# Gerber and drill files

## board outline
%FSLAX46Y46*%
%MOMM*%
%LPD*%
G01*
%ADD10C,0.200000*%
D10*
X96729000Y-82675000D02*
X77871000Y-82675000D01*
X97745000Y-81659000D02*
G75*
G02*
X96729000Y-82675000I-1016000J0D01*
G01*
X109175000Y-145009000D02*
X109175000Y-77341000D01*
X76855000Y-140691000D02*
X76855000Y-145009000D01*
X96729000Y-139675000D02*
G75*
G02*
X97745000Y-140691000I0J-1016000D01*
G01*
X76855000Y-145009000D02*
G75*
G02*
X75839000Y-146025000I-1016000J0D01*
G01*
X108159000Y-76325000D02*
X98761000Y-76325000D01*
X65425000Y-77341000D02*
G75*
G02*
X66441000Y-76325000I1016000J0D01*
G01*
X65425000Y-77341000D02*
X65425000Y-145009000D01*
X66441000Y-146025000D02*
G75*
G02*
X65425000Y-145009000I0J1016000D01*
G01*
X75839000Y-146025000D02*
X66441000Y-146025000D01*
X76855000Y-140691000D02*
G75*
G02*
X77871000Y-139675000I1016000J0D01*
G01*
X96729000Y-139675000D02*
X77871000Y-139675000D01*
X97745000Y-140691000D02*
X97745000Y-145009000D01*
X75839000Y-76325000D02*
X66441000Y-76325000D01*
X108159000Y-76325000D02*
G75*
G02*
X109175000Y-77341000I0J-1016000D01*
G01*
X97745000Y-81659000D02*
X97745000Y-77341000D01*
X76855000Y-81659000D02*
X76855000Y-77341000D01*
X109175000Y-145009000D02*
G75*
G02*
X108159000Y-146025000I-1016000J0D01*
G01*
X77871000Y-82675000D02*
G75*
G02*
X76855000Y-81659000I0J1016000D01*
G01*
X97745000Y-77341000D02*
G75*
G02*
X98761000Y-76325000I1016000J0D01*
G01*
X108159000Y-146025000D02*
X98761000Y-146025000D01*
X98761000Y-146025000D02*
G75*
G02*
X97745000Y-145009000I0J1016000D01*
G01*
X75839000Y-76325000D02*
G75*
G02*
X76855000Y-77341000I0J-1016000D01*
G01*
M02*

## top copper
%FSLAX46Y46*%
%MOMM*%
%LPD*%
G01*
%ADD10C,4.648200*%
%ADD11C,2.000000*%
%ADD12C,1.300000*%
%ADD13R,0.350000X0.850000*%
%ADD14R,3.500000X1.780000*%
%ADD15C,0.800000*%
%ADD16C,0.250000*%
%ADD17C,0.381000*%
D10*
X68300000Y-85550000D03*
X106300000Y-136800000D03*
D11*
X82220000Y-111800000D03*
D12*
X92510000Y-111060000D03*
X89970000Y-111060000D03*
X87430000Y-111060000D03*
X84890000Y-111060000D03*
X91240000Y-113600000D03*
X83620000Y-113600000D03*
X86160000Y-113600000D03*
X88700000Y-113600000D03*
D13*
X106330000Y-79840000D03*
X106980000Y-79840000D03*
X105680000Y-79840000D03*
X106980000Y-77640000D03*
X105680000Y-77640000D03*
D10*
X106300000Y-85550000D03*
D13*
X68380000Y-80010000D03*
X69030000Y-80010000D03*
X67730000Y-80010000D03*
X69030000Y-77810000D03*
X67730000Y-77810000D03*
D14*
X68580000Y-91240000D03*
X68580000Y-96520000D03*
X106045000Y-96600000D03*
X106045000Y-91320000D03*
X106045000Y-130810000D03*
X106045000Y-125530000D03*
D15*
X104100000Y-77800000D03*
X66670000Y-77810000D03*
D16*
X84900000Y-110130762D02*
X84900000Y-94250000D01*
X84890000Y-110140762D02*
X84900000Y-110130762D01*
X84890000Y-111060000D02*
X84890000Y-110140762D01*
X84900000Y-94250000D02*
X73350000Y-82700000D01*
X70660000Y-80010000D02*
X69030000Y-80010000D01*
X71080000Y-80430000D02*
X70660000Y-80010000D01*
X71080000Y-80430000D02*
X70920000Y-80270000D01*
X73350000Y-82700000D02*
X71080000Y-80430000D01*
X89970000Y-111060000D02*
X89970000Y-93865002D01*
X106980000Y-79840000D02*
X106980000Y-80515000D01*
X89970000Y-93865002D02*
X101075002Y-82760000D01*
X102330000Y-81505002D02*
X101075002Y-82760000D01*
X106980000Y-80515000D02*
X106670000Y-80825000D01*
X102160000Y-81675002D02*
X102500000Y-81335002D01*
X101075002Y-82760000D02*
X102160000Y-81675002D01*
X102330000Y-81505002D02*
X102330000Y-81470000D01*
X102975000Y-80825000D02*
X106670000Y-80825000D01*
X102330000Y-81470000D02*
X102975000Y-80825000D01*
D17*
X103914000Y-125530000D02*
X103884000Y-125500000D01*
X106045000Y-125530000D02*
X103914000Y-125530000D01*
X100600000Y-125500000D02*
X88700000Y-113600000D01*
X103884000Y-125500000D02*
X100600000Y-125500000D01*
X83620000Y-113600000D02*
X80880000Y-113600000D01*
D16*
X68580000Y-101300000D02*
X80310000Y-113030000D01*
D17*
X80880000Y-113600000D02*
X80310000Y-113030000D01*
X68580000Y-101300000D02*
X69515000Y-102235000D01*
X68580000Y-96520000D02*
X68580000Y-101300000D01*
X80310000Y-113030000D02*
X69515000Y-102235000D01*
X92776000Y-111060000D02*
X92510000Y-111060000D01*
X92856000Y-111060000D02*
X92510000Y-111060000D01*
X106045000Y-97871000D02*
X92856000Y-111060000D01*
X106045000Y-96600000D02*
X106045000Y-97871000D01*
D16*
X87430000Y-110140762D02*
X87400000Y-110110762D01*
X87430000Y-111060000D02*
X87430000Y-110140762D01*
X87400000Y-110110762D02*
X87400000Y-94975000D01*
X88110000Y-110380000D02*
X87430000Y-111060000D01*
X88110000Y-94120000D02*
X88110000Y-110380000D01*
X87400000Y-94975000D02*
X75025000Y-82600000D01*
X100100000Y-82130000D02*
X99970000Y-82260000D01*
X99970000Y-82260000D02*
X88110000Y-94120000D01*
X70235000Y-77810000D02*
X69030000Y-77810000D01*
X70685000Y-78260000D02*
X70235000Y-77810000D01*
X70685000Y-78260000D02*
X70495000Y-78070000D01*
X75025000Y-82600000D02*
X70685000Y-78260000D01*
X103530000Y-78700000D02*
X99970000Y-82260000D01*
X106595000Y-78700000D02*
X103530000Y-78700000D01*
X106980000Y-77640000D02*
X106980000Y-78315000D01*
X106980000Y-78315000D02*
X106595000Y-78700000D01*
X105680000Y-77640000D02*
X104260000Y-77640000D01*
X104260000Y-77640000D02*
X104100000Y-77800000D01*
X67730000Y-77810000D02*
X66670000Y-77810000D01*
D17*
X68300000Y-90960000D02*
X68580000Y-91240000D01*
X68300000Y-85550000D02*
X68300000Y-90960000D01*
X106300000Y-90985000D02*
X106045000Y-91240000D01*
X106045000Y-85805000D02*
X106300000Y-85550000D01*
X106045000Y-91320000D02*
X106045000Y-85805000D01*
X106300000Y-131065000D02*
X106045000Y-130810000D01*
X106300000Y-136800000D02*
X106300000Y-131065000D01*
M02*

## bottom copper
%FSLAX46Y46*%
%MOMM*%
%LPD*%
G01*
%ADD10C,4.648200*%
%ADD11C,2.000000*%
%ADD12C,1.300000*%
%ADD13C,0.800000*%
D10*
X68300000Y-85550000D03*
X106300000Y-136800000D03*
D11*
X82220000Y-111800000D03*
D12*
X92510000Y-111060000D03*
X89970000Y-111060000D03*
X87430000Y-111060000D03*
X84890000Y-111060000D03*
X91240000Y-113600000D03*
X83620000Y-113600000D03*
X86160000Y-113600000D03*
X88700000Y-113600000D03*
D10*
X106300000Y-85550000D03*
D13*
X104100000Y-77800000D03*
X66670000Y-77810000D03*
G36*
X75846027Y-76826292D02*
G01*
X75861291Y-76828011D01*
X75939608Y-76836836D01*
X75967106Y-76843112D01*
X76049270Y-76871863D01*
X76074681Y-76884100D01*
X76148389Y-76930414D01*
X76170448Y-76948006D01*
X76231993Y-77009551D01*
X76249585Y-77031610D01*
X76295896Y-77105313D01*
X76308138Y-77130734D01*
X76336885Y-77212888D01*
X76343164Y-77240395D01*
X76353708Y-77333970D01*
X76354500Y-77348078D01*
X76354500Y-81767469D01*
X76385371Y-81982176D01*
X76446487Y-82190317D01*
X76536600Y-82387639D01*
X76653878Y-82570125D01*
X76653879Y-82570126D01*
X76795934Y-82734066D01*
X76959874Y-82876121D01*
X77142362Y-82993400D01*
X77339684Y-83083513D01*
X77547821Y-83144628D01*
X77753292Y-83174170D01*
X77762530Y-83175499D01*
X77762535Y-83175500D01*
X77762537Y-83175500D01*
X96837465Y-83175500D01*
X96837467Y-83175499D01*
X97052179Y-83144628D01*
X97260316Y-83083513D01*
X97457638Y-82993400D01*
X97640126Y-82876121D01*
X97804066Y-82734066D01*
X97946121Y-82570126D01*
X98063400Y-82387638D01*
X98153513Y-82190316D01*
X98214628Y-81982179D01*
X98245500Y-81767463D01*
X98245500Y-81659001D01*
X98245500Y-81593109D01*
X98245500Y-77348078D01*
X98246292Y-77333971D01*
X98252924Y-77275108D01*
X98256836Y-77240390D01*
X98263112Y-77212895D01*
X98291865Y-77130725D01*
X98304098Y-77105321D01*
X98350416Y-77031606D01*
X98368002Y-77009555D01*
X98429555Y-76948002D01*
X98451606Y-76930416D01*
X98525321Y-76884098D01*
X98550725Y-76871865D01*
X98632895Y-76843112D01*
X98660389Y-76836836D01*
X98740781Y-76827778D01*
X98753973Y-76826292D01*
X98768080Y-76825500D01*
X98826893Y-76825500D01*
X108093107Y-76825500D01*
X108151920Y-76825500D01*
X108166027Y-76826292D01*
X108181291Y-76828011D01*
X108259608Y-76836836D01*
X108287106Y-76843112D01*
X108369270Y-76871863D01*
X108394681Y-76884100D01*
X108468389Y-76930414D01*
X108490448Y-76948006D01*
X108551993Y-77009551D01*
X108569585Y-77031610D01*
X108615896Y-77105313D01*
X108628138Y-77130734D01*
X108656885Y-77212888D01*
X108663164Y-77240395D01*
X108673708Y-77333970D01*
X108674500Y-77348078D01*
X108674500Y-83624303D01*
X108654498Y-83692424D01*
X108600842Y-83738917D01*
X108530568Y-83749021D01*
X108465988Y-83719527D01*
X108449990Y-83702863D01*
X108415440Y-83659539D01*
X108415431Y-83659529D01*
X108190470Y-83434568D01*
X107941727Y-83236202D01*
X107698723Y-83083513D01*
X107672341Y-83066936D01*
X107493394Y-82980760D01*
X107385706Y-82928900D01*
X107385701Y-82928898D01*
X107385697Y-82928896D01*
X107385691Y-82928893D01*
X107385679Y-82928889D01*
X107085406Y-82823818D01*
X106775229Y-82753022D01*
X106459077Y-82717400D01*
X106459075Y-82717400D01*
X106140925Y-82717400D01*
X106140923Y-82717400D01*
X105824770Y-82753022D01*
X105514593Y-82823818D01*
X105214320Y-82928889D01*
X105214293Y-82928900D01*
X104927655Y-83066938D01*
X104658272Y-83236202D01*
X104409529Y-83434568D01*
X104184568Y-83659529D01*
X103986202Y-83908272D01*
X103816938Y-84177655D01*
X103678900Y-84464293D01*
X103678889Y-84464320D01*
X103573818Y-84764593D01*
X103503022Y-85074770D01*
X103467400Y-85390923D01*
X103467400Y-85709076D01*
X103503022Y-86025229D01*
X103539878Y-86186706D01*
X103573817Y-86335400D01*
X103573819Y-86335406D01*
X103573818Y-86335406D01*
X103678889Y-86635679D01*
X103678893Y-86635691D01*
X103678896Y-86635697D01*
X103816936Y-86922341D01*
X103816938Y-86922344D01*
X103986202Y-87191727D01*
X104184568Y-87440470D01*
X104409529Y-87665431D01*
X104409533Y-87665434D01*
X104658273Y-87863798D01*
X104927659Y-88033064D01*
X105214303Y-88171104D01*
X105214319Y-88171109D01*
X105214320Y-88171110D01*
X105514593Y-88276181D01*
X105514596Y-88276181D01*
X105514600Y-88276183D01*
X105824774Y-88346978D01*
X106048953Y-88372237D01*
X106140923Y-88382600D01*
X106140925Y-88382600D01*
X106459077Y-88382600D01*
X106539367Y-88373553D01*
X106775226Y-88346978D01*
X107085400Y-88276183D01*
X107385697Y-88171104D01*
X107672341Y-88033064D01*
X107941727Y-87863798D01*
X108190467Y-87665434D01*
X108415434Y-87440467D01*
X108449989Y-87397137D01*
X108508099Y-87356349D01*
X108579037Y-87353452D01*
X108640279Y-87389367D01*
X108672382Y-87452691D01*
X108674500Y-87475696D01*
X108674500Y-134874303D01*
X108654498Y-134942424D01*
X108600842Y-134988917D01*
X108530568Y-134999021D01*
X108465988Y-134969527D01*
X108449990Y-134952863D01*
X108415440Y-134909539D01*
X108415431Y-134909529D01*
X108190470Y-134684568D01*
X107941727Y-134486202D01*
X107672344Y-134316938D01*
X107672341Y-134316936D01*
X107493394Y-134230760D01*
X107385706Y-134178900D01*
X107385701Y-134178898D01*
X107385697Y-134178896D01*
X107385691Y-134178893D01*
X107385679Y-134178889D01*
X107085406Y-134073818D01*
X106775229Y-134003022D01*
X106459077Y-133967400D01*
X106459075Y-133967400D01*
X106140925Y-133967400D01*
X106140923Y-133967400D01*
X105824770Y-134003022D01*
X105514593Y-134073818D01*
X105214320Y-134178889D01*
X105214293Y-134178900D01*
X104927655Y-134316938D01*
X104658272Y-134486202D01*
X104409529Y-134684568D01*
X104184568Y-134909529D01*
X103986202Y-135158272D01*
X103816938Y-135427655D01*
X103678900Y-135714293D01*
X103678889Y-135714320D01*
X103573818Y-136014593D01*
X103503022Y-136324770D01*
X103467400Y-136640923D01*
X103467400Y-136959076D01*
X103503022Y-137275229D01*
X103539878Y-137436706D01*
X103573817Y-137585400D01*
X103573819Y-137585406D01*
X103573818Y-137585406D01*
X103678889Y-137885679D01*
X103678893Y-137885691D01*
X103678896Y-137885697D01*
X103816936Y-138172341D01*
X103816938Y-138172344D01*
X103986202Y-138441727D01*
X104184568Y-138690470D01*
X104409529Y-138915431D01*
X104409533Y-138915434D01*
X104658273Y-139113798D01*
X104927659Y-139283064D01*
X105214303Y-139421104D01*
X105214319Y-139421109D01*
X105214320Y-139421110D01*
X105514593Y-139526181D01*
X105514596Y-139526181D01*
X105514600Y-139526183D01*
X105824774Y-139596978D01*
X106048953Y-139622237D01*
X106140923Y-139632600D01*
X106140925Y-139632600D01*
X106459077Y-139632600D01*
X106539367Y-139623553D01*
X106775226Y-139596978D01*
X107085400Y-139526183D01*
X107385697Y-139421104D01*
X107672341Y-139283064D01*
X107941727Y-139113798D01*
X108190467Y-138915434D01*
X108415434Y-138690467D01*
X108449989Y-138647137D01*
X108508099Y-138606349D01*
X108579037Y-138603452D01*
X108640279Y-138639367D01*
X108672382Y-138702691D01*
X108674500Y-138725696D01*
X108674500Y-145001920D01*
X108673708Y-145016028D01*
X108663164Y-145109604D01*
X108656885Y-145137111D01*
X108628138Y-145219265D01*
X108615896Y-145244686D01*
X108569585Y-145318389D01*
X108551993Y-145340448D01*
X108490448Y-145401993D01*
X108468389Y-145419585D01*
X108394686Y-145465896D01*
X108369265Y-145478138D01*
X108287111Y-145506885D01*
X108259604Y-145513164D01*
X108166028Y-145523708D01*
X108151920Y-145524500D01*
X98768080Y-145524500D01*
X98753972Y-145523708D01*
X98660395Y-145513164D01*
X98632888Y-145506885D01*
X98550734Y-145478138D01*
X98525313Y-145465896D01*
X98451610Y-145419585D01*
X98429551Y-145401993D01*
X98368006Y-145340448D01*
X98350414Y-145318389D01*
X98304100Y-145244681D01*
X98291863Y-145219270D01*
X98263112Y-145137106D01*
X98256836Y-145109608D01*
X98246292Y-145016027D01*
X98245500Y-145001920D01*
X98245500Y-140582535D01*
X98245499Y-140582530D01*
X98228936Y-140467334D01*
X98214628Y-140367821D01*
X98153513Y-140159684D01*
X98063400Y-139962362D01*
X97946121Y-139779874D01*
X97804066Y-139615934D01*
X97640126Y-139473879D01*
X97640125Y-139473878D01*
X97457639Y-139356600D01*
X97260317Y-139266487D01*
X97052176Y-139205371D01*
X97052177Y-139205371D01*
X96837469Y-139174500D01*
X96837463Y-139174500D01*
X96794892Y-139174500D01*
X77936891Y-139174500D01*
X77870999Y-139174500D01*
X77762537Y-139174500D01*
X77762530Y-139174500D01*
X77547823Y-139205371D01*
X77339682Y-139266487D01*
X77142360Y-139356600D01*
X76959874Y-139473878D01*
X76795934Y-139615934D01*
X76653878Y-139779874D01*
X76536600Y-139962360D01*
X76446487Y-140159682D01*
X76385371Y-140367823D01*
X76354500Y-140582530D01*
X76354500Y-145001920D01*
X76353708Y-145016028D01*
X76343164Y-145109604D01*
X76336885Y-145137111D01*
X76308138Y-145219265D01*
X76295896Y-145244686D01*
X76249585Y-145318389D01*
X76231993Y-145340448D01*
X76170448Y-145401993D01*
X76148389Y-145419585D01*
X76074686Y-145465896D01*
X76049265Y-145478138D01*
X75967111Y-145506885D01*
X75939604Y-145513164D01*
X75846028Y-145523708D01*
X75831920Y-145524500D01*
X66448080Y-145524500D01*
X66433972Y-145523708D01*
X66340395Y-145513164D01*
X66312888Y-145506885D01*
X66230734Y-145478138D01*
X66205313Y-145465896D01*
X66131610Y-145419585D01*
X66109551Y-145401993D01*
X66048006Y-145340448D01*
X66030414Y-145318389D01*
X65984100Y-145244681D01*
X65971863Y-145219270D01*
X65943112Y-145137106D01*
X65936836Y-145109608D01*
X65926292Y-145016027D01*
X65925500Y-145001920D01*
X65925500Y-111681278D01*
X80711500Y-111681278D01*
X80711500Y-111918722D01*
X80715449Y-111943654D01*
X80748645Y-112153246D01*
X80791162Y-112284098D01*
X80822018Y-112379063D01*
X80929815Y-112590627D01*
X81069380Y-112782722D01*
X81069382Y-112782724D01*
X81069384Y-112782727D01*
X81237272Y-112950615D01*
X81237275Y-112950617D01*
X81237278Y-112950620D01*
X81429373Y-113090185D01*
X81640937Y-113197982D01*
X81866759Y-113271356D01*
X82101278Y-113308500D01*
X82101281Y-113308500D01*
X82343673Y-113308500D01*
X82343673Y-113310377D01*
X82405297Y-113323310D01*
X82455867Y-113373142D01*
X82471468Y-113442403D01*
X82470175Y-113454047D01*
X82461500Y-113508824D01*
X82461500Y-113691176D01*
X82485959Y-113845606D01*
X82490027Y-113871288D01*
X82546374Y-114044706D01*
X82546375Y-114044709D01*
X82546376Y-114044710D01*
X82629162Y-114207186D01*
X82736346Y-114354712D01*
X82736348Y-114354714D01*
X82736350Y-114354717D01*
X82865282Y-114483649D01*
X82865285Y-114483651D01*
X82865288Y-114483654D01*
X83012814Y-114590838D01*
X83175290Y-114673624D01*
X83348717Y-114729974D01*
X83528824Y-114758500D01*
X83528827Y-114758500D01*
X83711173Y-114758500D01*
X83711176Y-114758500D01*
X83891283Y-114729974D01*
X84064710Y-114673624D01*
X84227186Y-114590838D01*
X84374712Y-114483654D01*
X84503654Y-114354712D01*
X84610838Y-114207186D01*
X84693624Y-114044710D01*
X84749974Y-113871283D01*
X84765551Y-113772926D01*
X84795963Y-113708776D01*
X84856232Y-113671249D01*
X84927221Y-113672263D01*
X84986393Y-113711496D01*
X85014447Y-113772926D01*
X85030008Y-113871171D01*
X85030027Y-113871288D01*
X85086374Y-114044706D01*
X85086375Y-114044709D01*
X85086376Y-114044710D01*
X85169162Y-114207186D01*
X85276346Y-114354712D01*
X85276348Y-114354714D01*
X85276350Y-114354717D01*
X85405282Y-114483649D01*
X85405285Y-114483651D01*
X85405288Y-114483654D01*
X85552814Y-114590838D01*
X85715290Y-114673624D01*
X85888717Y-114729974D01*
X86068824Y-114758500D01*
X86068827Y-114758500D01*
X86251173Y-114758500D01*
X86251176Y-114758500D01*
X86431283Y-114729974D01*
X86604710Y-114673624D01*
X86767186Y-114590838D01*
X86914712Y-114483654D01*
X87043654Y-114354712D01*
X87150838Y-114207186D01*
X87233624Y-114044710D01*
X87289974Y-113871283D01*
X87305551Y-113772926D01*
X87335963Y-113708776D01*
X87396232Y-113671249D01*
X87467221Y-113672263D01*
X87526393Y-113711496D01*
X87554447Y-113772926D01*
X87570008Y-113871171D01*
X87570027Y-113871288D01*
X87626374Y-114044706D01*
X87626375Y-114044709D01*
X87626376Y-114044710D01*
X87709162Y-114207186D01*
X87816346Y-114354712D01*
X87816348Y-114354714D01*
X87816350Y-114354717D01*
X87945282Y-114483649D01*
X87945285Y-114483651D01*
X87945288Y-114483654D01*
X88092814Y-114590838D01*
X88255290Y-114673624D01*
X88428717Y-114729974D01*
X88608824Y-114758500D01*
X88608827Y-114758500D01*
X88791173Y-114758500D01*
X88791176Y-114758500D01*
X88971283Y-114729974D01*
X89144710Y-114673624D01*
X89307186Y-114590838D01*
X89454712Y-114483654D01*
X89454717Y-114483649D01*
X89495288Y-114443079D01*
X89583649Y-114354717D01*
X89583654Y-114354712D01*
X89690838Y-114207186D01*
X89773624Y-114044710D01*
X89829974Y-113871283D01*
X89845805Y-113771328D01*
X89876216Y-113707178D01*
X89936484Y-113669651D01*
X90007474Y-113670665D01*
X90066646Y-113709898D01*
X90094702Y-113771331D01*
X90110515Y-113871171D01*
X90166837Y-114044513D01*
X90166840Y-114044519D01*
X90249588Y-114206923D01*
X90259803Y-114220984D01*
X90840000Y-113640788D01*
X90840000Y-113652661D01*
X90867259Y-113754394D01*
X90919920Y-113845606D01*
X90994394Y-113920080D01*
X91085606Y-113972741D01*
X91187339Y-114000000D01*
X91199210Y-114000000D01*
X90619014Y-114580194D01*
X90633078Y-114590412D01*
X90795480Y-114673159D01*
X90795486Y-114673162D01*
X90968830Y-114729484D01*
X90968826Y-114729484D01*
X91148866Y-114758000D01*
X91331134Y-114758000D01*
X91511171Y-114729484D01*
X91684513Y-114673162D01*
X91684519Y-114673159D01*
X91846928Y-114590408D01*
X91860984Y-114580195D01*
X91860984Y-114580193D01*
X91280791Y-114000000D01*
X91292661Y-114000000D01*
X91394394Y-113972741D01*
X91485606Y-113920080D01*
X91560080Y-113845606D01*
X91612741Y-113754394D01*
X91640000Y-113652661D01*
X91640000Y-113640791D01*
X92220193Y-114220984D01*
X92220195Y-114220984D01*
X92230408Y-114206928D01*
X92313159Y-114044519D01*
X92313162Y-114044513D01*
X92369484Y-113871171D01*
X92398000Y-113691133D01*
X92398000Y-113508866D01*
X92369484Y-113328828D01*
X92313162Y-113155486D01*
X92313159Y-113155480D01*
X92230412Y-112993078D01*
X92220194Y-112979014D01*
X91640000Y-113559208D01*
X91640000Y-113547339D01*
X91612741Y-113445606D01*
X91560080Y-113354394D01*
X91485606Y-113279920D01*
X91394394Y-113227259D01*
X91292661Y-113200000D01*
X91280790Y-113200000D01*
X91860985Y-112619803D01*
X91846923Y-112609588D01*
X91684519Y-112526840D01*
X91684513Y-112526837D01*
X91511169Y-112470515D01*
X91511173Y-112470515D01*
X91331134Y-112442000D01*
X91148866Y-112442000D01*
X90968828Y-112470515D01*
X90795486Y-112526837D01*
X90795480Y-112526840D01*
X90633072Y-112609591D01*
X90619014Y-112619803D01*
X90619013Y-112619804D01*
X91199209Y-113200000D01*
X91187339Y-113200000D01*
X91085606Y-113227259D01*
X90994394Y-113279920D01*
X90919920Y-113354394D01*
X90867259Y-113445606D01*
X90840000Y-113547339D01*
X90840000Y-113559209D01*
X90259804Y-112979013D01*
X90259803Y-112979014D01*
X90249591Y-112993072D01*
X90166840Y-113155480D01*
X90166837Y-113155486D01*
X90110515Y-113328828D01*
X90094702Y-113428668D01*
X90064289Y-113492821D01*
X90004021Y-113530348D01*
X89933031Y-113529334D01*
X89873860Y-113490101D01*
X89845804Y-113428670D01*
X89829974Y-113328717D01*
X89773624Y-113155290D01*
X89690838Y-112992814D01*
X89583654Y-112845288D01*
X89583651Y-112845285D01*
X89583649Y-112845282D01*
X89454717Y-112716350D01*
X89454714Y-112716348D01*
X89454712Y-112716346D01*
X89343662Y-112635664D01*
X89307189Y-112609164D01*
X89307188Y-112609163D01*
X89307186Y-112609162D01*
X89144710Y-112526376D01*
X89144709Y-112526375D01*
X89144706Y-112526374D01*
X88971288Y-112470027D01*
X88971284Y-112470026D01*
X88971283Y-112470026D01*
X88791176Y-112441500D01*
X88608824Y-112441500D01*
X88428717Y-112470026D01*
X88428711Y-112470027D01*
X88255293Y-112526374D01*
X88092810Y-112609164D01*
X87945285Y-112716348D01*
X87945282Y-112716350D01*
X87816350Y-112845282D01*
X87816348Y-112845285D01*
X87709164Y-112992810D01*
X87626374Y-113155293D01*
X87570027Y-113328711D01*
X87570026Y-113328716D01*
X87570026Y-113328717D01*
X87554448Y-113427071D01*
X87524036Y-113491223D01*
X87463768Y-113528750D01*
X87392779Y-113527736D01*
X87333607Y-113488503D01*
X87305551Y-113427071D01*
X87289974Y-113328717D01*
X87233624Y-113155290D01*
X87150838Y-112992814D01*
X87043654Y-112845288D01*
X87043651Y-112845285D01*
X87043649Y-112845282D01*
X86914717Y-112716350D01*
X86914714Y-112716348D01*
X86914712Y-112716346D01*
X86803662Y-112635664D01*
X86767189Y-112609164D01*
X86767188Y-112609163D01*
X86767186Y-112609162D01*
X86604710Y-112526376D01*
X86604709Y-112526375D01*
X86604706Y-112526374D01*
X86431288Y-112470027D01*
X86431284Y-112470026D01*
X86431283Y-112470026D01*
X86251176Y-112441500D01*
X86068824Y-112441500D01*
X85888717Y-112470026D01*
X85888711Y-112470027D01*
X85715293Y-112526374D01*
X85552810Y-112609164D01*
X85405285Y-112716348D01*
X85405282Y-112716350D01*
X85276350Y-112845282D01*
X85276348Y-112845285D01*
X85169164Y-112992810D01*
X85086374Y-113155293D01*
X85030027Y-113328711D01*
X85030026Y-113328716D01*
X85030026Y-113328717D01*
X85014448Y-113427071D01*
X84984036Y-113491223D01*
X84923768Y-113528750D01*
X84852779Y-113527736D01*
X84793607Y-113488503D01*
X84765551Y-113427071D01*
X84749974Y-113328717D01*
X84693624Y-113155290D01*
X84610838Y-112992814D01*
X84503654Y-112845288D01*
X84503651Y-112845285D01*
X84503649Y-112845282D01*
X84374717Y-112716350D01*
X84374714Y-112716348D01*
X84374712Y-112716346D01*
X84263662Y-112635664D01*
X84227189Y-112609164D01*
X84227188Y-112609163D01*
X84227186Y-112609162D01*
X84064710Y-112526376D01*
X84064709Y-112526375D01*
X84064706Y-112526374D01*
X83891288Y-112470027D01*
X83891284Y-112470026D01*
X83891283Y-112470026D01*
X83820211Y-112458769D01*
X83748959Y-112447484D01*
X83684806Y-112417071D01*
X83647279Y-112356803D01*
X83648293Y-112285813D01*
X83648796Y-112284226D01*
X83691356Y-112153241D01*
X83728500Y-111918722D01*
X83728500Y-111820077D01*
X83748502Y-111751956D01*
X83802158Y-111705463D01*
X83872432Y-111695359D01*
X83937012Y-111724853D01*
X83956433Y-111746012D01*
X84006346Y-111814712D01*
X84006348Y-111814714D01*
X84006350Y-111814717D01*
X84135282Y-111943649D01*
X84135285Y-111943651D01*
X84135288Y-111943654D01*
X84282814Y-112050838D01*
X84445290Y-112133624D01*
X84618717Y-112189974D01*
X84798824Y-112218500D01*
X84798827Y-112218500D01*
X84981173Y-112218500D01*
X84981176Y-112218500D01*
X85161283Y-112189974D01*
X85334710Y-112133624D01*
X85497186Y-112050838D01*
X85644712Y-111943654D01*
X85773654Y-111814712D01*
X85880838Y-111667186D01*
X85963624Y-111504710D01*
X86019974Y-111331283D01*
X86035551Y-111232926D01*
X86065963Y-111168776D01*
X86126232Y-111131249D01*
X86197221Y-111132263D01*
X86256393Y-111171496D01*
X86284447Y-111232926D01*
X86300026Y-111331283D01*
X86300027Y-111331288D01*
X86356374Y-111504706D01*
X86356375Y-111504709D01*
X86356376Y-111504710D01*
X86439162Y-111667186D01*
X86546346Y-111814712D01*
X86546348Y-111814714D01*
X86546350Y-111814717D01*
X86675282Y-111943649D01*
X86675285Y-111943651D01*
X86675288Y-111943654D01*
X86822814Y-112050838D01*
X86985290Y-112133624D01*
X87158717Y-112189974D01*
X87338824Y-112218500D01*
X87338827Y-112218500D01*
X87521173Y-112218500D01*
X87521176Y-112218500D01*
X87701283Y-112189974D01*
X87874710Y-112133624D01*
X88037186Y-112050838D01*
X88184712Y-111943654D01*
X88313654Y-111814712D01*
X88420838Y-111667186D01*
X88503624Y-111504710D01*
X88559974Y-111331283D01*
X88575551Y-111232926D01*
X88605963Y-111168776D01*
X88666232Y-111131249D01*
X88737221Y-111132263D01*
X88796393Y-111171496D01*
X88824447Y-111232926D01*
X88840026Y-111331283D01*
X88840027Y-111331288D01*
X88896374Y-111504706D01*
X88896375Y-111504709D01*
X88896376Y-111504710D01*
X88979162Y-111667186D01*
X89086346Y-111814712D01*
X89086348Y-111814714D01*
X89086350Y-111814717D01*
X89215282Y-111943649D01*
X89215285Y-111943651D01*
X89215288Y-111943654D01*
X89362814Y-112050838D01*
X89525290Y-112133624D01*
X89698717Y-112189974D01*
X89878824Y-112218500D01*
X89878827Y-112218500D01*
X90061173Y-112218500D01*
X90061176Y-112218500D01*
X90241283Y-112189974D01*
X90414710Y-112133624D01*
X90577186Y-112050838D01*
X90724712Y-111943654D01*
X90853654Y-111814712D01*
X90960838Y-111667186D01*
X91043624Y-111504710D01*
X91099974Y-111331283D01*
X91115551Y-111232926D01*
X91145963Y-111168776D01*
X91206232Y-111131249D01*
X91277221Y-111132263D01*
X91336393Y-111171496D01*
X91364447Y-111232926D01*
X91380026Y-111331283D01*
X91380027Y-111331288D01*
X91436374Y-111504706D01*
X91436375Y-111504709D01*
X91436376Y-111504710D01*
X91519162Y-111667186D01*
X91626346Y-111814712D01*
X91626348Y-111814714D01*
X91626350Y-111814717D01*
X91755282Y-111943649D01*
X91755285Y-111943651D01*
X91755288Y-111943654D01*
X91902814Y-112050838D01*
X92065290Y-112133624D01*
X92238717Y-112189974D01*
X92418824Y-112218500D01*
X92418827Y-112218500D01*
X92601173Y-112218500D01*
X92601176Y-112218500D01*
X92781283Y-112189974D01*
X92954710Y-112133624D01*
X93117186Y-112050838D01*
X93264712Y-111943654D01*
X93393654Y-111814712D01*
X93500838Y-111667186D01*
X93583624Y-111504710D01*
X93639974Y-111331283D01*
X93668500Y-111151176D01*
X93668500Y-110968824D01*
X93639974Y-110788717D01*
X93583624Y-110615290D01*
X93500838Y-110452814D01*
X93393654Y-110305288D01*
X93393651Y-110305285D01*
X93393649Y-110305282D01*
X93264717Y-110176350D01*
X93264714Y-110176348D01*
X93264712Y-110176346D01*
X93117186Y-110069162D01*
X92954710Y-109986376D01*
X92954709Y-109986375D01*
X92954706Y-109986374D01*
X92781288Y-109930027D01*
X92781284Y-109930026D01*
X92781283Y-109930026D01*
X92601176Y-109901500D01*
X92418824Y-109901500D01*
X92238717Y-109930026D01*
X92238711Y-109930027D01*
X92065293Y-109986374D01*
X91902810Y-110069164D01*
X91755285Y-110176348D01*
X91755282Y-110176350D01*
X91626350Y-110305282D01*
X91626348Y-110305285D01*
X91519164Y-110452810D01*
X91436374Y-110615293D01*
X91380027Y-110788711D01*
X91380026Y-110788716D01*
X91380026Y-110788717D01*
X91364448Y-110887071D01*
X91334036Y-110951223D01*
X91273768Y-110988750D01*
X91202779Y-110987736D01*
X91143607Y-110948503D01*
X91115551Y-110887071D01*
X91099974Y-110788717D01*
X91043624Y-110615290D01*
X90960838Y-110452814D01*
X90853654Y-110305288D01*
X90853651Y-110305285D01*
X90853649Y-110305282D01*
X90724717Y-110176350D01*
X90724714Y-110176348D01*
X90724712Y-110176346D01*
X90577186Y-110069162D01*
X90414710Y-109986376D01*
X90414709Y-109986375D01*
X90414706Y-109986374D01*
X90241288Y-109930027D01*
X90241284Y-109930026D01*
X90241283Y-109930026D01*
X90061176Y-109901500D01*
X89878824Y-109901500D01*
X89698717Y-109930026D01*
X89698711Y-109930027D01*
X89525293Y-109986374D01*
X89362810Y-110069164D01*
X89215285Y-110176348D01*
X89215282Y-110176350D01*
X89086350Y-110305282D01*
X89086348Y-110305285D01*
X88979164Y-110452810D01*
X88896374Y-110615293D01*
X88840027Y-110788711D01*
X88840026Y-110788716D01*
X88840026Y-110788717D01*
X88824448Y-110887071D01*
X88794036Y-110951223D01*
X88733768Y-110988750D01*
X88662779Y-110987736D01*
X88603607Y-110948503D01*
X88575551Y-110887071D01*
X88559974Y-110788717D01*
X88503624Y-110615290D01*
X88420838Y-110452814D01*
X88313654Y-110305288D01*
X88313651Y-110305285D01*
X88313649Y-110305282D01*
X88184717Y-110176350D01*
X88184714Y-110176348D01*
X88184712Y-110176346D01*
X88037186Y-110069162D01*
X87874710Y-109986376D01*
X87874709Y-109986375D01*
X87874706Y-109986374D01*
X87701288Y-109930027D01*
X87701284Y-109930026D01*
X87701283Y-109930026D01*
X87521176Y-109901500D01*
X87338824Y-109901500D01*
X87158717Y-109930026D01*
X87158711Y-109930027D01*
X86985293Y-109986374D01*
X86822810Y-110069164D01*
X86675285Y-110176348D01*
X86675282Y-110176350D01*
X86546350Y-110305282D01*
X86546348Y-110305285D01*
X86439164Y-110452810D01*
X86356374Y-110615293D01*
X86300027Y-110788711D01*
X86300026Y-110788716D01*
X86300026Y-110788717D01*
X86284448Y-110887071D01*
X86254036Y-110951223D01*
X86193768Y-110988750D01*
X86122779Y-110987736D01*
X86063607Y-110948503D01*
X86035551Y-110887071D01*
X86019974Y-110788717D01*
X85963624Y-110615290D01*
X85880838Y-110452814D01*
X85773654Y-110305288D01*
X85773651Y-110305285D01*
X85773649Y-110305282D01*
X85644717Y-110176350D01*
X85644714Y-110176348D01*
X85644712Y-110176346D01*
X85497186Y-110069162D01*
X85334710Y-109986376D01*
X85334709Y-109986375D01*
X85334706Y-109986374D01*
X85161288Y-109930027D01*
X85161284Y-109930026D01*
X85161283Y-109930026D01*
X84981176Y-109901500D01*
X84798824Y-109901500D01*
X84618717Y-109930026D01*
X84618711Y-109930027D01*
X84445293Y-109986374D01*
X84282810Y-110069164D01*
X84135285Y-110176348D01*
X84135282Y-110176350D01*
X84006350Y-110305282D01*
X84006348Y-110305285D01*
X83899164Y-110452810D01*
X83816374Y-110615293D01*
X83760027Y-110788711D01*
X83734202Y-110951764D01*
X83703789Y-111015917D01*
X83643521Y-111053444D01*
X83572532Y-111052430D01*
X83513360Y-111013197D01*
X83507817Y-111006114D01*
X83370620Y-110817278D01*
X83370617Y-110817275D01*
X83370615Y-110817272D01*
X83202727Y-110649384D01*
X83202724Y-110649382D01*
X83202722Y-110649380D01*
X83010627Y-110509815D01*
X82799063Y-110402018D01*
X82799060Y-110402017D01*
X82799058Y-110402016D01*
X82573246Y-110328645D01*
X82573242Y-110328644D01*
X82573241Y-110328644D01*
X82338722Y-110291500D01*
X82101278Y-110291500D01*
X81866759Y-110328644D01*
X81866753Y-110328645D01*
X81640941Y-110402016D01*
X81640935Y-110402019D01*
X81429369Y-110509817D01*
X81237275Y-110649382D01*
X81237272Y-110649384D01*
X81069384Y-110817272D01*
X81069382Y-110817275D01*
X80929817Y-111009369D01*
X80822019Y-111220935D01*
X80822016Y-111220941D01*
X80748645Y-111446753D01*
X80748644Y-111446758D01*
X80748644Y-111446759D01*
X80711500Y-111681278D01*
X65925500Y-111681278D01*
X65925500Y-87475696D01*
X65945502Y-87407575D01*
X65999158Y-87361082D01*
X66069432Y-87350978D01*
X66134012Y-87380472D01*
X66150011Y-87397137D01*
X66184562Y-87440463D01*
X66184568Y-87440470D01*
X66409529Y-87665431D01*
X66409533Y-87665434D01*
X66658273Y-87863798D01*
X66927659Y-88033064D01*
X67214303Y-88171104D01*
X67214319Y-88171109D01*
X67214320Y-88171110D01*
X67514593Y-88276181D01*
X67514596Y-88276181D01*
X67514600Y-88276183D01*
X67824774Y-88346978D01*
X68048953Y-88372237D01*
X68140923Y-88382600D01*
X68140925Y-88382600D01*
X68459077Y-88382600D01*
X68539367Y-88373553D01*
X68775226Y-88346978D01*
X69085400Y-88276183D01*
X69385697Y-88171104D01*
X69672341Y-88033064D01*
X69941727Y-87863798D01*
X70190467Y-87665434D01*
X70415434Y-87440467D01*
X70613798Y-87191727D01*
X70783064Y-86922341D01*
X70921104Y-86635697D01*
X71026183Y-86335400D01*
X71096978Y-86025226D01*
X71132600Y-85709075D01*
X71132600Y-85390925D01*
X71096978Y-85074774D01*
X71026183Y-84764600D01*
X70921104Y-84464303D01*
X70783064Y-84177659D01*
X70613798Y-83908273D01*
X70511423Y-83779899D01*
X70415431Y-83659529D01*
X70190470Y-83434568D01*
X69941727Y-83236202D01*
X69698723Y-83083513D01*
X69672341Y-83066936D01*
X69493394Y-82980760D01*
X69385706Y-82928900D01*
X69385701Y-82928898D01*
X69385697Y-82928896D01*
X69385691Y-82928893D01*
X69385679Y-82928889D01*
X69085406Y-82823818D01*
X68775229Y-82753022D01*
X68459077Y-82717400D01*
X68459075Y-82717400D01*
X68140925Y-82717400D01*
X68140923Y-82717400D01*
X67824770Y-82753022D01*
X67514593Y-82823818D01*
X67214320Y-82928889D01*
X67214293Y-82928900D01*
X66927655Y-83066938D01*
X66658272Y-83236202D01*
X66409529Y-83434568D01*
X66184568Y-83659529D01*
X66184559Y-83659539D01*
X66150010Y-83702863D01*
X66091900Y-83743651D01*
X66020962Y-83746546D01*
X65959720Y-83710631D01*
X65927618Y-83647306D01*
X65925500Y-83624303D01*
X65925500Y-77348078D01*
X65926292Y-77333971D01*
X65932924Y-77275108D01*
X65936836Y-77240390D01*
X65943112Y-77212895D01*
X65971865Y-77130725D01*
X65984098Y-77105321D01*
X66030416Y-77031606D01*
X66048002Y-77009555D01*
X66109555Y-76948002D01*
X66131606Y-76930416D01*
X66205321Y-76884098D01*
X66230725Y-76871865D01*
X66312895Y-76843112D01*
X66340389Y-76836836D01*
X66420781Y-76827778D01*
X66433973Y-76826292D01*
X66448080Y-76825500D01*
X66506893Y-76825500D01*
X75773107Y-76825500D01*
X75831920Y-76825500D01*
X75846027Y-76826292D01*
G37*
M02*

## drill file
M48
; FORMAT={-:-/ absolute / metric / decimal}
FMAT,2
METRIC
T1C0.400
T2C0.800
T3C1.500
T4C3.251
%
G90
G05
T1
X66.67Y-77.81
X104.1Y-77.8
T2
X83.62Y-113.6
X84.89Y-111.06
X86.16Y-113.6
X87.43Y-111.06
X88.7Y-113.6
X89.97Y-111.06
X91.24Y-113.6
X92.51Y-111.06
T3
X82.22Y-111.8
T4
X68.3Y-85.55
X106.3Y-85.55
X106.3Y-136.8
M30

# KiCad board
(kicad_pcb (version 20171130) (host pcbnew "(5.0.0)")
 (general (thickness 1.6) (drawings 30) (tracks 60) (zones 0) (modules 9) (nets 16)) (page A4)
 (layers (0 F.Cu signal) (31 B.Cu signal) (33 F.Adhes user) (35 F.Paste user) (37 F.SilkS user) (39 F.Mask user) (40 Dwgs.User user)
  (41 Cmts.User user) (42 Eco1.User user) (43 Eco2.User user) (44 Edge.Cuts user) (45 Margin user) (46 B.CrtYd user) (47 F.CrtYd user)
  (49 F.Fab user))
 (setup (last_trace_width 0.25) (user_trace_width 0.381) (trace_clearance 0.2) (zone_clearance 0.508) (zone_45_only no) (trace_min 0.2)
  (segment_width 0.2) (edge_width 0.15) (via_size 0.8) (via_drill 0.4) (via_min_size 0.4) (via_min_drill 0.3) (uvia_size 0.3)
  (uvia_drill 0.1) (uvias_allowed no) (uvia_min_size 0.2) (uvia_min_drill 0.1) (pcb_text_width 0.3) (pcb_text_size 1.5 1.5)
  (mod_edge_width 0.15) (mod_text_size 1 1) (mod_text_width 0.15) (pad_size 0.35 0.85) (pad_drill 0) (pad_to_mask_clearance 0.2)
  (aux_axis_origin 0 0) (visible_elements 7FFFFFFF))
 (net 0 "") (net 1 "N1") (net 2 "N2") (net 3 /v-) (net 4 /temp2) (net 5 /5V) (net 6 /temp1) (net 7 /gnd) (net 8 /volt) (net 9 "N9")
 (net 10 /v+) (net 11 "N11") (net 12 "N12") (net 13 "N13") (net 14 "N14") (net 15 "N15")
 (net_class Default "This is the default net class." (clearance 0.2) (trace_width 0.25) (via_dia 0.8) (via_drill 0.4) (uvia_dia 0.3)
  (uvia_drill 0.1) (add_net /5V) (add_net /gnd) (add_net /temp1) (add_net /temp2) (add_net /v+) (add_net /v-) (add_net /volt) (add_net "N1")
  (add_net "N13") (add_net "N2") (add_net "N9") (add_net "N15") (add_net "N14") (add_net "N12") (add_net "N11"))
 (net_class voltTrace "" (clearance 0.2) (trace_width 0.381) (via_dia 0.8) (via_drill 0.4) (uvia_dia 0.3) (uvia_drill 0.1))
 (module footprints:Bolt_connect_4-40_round (layer F.Cu) (at 68.3 85.55)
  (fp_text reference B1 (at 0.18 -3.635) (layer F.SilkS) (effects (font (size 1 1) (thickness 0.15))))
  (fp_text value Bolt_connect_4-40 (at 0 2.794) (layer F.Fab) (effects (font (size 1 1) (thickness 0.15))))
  (pad 1 thru_hole circle (at 0 0) (size 4.6482 4.6482) (drill 3.2512) (layers *.Cu *.Mask) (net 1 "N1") (clearance 0.508)))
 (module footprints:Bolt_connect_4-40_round (layer F.Cu) (at 106.3 136.8)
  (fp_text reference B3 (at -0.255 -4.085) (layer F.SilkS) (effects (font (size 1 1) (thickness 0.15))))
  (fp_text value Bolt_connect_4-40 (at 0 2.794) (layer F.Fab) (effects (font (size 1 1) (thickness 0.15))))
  (pad 1 thru_hole circle (at 0 0) (size 4.6482 4.6482) (drill 3.2512) (layers *.Cu *.Mask) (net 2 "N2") (clearance 0.508)))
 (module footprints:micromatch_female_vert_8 (layer F.Cu) (at 88.7 113.6 90)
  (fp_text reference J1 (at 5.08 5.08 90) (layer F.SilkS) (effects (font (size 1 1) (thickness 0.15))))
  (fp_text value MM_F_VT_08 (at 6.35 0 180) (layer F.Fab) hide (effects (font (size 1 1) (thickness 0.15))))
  (pad 9 thru_hole circle (at 1.8 -6.48 90) (size 2 2) (drill 1.5) (layers *.Cu *.Mask))
  (pad 8 thru_hole circle (at 2.54 3.81 90) (size 1.3 1.3) (drill 0.8) (layers *.Cu *.Mask) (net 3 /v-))
  (pad 6 thru_hole circle (at 2.54 1.27 90) (size 1.3 1.3) (drill 0.8) (layers *.Cu *.Mask) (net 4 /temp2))
  (pad 4 thru_hole circle (at 2.54 -1.27 90) (size 1.3 1.3) (drill 0.8) (layers *.Cu *.Mask) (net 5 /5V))
  (pad 2 thru_hole circle (at 2.54 -3.81 90) (size 1.3 1.3) (drill 0.8) (layers *.Cu *.Mask) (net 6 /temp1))
  (pad 7 thru_hole circle (at 0 2.54 90) (size 1.3 1.3) (drill 0.8) (layers *.Cu *.Mask) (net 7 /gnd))
  (pad 1 thru_hole circle (at 0 -5.08 90) (size 1.3 1.3) (drill 0.8) (layers *.Cu *.Mask) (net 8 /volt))
  (pad 3 thru_hole circle (at 0 -2.54 90) (size 1.3 1.3) (drill 0.8) (layers *.Cu *.Mask) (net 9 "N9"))
  (pad 5 thru_hole circle (at 0 0 90) (size 1.3 1.3) (drill 0.8) (layers *.Cu *.Mask) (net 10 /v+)))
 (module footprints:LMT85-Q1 (layer F.Cu) (at 105.68 79.84)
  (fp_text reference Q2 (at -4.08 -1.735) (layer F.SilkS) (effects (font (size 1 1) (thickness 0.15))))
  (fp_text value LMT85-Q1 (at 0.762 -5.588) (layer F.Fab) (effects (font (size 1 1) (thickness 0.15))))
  (pad 3 smd rect (at 0.65 0) (size 0.35 0.85) (layers F.Cu F.Paste F.Mask) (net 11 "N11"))
  (pad 4 smd rect (at 1.3 0) (size 0.35 0.85) (layers F.Cu F.Paste F.Mask) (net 4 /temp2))
  (pad 2 smd rect (at 0 0) (size 0.35 0.85) (layers F.Cu F.Paste F.Mask) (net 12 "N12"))
  (pad 5 smd rect (at 1.3 -2.2) (size 0.35 0.85) (layers F.Cu F.Paste F.Mask) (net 5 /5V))
  (pad 1 smd rect (at 0 -2.2) (size 0.35 0.85) (layers F.Cu F.Paste F.Mask) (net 7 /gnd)))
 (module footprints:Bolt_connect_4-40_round (layer F.Cu) (at 106.3 85.55)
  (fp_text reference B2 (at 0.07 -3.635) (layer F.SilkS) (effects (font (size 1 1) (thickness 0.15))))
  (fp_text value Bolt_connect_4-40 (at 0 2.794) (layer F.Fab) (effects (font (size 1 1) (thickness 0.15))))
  (pad 1 thru_hole circle (at 0 0) (size 4.6482 4.6482) (drill 3.2512) (layers *.Cu *.Mask) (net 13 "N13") (clearance 0.508)))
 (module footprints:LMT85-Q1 (layer F.Cu) (at 67.73 80.01)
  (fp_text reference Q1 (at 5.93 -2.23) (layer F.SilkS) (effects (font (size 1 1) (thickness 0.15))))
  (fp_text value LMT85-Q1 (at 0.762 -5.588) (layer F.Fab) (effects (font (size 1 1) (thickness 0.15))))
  (pad 3 smd rect (at 0.65 0) (size 0.35 0.85) (layers F.Cu F.Paste F.Mask) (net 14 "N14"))
  (pad 4 smd rect (at 1.3 0) (size 0.35 0.85) (layers F.Cu F.Paste F.Mask) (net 6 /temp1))
  (pad 2 smd rect (at 0 0) (size 0.35 0.85) (layers F.Cu F.Paste F.Mask) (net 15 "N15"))
  (pad 5 smd rect (at 1.3 -2.2) (size 0.35 0.85) (layers F.Cu F.Paste F.Mask) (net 5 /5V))
  (pad 1 smd rect (at 0 -2.2) (size 0.35 0.85) (layers F.Cu F.Paste F.Mask) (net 7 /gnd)))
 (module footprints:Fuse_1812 (layer F.Cu) (at 68.58 96.52 90)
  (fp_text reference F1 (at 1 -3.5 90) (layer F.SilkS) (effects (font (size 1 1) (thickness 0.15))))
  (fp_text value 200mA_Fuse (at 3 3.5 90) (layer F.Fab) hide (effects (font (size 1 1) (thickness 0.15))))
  (pad 2 smd rect (at 5.28 0 90) (size 1.78 3.5) (layers F.Cu F.Paste F.Mask) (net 1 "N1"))
  (pad 1 smd rect (at 0 0 90) (size 1.78 3.5) (layers F.Cu F.Paste F.Mask) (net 8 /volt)))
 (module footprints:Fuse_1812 (layer F.Cu) (at 106.045 96.6 90)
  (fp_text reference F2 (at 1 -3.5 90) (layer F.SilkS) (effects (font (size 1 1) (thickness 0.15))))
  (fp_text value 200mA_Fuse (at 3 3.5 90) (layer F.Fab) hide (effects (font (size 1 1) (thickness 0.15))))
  (pad 1 smd rect (at 0 0 90) (size 1.78 3.5) (layers F.Cu F.Paste F.Mask) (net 3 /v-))
  (pad 2 smd rect (at 5.28 0 90) (size 1.78 3.5) (layers F.Cu F.Paste F.Mask) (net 13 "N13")))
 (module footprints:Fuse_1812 (layer F.Cu) (at 106.045 125.53 270)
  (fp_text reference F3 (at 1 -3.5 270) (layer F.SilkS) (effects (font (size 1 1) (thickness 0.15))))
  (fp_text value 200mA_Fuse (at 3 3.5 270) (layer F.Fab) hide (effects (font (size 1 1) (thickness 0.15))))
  (pad 2 smd rect (at 5.28 0 270) (size 1.78 3.5) (layers F.Cu F.Paste F.Mask) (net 2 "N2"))
  (pad 1 smd rect (at 0 0 270) (size 1.78 3.5) (layers F.Cu F.Paste F.Mask) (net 10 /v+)))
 (gr_line (start 96.729 82.675) (end 77.871 82.675) (layer Edge.Cuts) (width 0.2))
 (gr_arc (start 96.729 81.659) (end 96.729 82.675) (angle -90) (layer Edge.Cuts) (width 0.2))
 (gr_line (start 109.175 145.009) (end 109.175 77.341) (layer Edge.Cuts) (width 0.2))
 (gr_line (start 76.855 140.691) (end 76.855 145.009) (layer Edge.Cuts) (width 0.2))
 (gr_arc (start 96.729 140.691) (end 97.745 140.691) (angle -90) (layer Edge.Cuts) (width 0.2))
 (gr_arc (start 75.839 145.009) (end 75.839 146.025) (angle -90) (layer Edge.Cuts) (width 0.2))
 (gr_line (start 108.159 76.325) (end 98.761 76.325) (layer Edge.Cuts) (width 0.2))
 (gr_arc (start 66.441 77.341) (end 66.441 76.325) (angle -90) (layer Edge.Cuts) (width 0.2))
 (gr_line (start 65.425 77.341) (end 65.425 145.009) (layer Edge.Cuts) (width 0.2))
 (gr_arc (start 66.441 145.009) (end 65.425 145.009) (angle -90) (layer Edge.Cuts) (width 0.2))
 (gr_line (start 75.839 146.025) (end 66.441 146.025) (layer Edge.Cuts) (width 0.2))
 (gr_arc (start 77.871 140.691) (end 77.871 139.675) (angle -90) (layer Edge.Cuts) (width 0.2))
 (gr_line (start 96.729 139.675) (end 77.871 139.675) (layer Edge.Cuts) (width 0.2))
 (gr_line (start 97.745 140.691) (end 97.745 145.009) (layer Edge.Cuts) (width 0.2))
 (gr_line (start 75.839 76.325) (end 66.441 76.325) (layer Edge.Cuts) (width 0.2))
 (gr_arc (start 108.159 77.341) (end 109.175 77.341) (angle -90) (layer Edge.Cuts) (width 0.2))
 (gr_line (start 97.745 81.659) (end 97.745 77.341) (layer Edge.Cuts) (width 0.2))
 (gr_line (start 76.855 81.659) (end 76.855 77.341) (layer Edge.Cuts) (width 0.2))
 (gr_arc (start 108.159 145.009) (end 108.159 146.025) (angle -90) (layer Edge.Cuts) (width 0.2))
 (gr_arc (start 77.871 81.659) (end 76.855 81.659) (angle -90) (layer Edge.Cuts) (width 0.2))
 (gr_arc (start 98.761 77.341) (end 98.761 76.325) (angle -90) (layer Edge.Cuts) (width 0.2))
 (gr_line (start 108.159 146.025) (end 98.761 146.025) (layer Edge.Cuts) (width 0.2))
 (gr_arc (start 98.761 145.009) (end 97.745 145.009) (angle -90) (layer Edge.Cuts) (width 0.2))
 (gr_arc (start 75.839 77.341) (end 76.855 77.341) (angle -90) (layer Edge.Cuts) (width 0.2))
 (segment (start 84.9 110.130762) (end 84.9 94.25) (width 0.25) (layer F.Cu) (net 6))
 (segment (start 84.89 110.140762) (end 84.9 110.130762) (width 0.25) (layer F.Cu) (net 6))
 (segment (start 84.89 111.06) (end 84.89 110.140762) (width 0.25) (layer F.Cu) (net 6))
 (segment (start 84.9 94.25) (end 73.35 82.7) (width 0.25) (layer F.Cu) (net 6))
 (segment (start 70.66 80.01) (end 69.03 80.01) (width 0.25) (layer F.Cu) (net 6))
 (segment (start 71.08 80.43) (end 70.66 80.01) (width 0.25) (layer F.Cu) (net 6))
 (segment (start 71.08 80.43) (end 70.92 80.27) (width 0.25) (layer F.Cu) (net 6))
 (segment (start 73.35 82.7) (end 71.08 80.43) (width 0.25) (layer F.Cu) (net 6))
 (segment (start 89.97 111.06) (end 89.97 93.865002) (width 0.25) (layer F.Cu) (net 4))
 (segment (start 106.98 79.84) (end 106.98 80.515) (width 0.25) (layer F.Cu) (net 4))
 (segment (start 89.97 93.865002) (end 101.075002 82.76) (width 0.25) (layer F.Cu) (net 4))
 (segment (start 102.33 81.505002) (end 101.075002 82.76) (width 0.25) (layer F.Cu) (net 4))
 (segment (start 106.98 80.515) (end 106.67 80.825) (width 0.25) (layer F.Cu) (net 4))
 (segment (start 102.16 81.675002) (end 102.5 81.335002) (width 0.25) (layer F.Cu) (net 4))
 (segment (start 101.075002 82.76) (end 102.16 81.675002) (width 0.25) (layer F.Cu) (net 4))
 (segment (start 102.33 81.505002) (end 102.33 81.47) (width 0.25) (layer F.Cu) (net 4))
 (segment (start 102.975 80.825) (end 106.67 80.825) (width 0.25) (layer F.Cu) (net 4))
 (segment (start 102.33 81.47) (end 102.975 80.825) (width 0.25) (layer F.Cu) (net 4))
 (segment (start 103.914 125.53) (end 103.884 125.5) (width 0.381) (layer F.Cu) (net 10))
 (segment (start 106.045 125.53) (end 103.914 125.53) (width 0.381) (layer F.Cu) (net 10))
 (segment (start 100.6 125.5) (end 88.7 113.6) (width 0.381) (layer F.Cu) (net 10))
 (segment (start 103.884 125.5) (end 100.6 125.5) (width 0.381) (layer F.Cu) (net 10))
 (segment (start 83.62 113.6) (end 80.88 113.6) (width 0.381) (layer F.Cu) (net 8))
 (segment (start 68.58 101.3) (end 80.31 113.03) (width 0.25) (layer F.Cu) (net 8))
 (segment (start 80.88 113.6) (end 80.31 113.03) (width 0.381) (layer F.Cu) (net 8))
 (segment (start 68.58 101.3) (end 69.515 102.235) (width 0.381) (layer F.Cu) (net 8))
 (segment (start 68.58 96.52) (end 68.58 101.3) (width 0.381) (layer F.Cu) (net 8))
 (segment (start 80.31 113.03) (end 69.515 102.235) (width 0.381) (layer F.Cu) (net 8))
 (segment (start 92.776 111.06) (end 92.51 111.06) (width 0.381) (layer F.Cu) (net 3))
 (segment (start 92.856 111.06) (end 92.51 111.06) (width 0.381) (layer F.Cu) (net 3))
 (segment (start 106.045 97.871) (end 92.856 111.06) (width 0.381) (layer F.Cu) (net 3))
 (segment (start 106.045 96.6) (end 106.045 97.871) (width 0.381) (layer F.Cu) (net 3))
 (segment (start 87.43 110.140762) (end 87.4 110.110762) (width 0.25) (layer F.Cu) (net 5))
 (segment (start 87.43 111.06) (end 87.43 110.140762) (width 0.25) (layer F.Cu) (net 5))
 (segment (start 87.4 110.110762) (end 87.4 94.975) (width 0.25) (layer F.Cu) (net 5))
 (segment (start 88.11 110.38) (end 87.43 111.06) (width 0.25) (layer F.Cu) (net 5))
 (segment (start 88.11 94.12) (end 88.11 110.38) (width 0.25) (layer F.Cu) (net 5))
 (segment (start 87.4 94.975) (end 75.025 82.6) (width 0.25) (layer F.Cu) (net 5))
 (segment (start 100.1 82.13) (end 99.97 82.26) (width 0.25) (layer F.Cu) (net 5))
 (segment (start 99.97 82.26) (end 88.11 94.12) (width 0.25) (layer F.Cu) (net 5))
 (segment (start 70.235 77.81) (end 69.03 77.81) (width 0.25) (layer F.Cu) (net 5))
 (segment (start 70.685 78.26) (end 70.235 77.81) (width 0.25) (layer F.Cu) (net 5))
 (segment (start 70.685 78.26) (end 70.495 78.07) (width 0.25) (layer F.Cu) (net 5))
 (segment (start 75.025 82.6) (end 70.685 78.26) (width 0.25) (layer F.Cu) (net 5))
 (segment (start 103.53 78.7) (end 99.97 82.26) (width 0.25) (layer F.Cu) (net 5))
 (segment (start 106.595 78.7) (end 103.53 78.7) (width 0.25) (layer F.Cu) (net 5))
 (segment (start 106.98 77.64) (end 106.98 78.315) (width 0.25) (layer F.Cu) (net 5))
 (segment (start 106.98 78.315) (end 106.595 78.7) (width 0.25) (layer F.Cu) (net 5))
 (via (at 104.1 77.8) (size 0.8) (drill 0.4) (layers F.Cu B.Cu) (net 7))
 (segment (start 105.68 77.64) (end 104.26 77.64) (width 0.25) (layer F.Cu) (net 7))
 (segment (start 104.26 77.64) (end 104.1 77.8) (width 0.25) (layer F.Cu) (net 7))
 (via (at 66.67 77.81) (size 0.8) (drill 0.4) (layers F.Cu B.Cu) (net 7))
 (segment (start 67.73 77.81) (end 66.67 77.81) (width 0.25) (layer F.Cu) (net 7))
 (segment (start 68.3 90.96) (end 68.58 91.24) (width 0.381) (layer F.Cu) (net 1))
 (segment (start 68.3 85.55) (end 68.3 90.96) (width 0.381) (layer F.Cu) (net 1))
 (segment (start 106.3 90.985) (end 106.045 91.24) (width 0.381) (layer F.Cu) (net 13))
 (segment (start 106.045 85.805) (end 106.3 85.55) (width 0.381) (layer F.Cu) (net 13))
 (segment (start 106.045 91.32) (end 106.045 85.805) (width 0.381) (layer F.Cu) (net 13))
 (segment (start 106.3 131.065) (end 106.045 130.81) (width 0.381) (layer F.Cu) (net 2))
 (segment (start 106.3 136.8) (end 106.3 131.065) (width 0.381) (layer F.Cu) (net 2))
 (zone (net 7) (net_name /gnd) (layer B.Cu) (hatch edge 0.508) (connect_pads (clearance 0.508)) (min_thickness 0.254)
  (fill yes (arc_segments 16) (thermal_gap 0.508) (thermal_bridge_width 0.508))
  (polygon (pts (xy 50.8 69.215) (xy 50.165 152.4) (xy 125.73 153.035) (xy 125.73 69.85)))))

